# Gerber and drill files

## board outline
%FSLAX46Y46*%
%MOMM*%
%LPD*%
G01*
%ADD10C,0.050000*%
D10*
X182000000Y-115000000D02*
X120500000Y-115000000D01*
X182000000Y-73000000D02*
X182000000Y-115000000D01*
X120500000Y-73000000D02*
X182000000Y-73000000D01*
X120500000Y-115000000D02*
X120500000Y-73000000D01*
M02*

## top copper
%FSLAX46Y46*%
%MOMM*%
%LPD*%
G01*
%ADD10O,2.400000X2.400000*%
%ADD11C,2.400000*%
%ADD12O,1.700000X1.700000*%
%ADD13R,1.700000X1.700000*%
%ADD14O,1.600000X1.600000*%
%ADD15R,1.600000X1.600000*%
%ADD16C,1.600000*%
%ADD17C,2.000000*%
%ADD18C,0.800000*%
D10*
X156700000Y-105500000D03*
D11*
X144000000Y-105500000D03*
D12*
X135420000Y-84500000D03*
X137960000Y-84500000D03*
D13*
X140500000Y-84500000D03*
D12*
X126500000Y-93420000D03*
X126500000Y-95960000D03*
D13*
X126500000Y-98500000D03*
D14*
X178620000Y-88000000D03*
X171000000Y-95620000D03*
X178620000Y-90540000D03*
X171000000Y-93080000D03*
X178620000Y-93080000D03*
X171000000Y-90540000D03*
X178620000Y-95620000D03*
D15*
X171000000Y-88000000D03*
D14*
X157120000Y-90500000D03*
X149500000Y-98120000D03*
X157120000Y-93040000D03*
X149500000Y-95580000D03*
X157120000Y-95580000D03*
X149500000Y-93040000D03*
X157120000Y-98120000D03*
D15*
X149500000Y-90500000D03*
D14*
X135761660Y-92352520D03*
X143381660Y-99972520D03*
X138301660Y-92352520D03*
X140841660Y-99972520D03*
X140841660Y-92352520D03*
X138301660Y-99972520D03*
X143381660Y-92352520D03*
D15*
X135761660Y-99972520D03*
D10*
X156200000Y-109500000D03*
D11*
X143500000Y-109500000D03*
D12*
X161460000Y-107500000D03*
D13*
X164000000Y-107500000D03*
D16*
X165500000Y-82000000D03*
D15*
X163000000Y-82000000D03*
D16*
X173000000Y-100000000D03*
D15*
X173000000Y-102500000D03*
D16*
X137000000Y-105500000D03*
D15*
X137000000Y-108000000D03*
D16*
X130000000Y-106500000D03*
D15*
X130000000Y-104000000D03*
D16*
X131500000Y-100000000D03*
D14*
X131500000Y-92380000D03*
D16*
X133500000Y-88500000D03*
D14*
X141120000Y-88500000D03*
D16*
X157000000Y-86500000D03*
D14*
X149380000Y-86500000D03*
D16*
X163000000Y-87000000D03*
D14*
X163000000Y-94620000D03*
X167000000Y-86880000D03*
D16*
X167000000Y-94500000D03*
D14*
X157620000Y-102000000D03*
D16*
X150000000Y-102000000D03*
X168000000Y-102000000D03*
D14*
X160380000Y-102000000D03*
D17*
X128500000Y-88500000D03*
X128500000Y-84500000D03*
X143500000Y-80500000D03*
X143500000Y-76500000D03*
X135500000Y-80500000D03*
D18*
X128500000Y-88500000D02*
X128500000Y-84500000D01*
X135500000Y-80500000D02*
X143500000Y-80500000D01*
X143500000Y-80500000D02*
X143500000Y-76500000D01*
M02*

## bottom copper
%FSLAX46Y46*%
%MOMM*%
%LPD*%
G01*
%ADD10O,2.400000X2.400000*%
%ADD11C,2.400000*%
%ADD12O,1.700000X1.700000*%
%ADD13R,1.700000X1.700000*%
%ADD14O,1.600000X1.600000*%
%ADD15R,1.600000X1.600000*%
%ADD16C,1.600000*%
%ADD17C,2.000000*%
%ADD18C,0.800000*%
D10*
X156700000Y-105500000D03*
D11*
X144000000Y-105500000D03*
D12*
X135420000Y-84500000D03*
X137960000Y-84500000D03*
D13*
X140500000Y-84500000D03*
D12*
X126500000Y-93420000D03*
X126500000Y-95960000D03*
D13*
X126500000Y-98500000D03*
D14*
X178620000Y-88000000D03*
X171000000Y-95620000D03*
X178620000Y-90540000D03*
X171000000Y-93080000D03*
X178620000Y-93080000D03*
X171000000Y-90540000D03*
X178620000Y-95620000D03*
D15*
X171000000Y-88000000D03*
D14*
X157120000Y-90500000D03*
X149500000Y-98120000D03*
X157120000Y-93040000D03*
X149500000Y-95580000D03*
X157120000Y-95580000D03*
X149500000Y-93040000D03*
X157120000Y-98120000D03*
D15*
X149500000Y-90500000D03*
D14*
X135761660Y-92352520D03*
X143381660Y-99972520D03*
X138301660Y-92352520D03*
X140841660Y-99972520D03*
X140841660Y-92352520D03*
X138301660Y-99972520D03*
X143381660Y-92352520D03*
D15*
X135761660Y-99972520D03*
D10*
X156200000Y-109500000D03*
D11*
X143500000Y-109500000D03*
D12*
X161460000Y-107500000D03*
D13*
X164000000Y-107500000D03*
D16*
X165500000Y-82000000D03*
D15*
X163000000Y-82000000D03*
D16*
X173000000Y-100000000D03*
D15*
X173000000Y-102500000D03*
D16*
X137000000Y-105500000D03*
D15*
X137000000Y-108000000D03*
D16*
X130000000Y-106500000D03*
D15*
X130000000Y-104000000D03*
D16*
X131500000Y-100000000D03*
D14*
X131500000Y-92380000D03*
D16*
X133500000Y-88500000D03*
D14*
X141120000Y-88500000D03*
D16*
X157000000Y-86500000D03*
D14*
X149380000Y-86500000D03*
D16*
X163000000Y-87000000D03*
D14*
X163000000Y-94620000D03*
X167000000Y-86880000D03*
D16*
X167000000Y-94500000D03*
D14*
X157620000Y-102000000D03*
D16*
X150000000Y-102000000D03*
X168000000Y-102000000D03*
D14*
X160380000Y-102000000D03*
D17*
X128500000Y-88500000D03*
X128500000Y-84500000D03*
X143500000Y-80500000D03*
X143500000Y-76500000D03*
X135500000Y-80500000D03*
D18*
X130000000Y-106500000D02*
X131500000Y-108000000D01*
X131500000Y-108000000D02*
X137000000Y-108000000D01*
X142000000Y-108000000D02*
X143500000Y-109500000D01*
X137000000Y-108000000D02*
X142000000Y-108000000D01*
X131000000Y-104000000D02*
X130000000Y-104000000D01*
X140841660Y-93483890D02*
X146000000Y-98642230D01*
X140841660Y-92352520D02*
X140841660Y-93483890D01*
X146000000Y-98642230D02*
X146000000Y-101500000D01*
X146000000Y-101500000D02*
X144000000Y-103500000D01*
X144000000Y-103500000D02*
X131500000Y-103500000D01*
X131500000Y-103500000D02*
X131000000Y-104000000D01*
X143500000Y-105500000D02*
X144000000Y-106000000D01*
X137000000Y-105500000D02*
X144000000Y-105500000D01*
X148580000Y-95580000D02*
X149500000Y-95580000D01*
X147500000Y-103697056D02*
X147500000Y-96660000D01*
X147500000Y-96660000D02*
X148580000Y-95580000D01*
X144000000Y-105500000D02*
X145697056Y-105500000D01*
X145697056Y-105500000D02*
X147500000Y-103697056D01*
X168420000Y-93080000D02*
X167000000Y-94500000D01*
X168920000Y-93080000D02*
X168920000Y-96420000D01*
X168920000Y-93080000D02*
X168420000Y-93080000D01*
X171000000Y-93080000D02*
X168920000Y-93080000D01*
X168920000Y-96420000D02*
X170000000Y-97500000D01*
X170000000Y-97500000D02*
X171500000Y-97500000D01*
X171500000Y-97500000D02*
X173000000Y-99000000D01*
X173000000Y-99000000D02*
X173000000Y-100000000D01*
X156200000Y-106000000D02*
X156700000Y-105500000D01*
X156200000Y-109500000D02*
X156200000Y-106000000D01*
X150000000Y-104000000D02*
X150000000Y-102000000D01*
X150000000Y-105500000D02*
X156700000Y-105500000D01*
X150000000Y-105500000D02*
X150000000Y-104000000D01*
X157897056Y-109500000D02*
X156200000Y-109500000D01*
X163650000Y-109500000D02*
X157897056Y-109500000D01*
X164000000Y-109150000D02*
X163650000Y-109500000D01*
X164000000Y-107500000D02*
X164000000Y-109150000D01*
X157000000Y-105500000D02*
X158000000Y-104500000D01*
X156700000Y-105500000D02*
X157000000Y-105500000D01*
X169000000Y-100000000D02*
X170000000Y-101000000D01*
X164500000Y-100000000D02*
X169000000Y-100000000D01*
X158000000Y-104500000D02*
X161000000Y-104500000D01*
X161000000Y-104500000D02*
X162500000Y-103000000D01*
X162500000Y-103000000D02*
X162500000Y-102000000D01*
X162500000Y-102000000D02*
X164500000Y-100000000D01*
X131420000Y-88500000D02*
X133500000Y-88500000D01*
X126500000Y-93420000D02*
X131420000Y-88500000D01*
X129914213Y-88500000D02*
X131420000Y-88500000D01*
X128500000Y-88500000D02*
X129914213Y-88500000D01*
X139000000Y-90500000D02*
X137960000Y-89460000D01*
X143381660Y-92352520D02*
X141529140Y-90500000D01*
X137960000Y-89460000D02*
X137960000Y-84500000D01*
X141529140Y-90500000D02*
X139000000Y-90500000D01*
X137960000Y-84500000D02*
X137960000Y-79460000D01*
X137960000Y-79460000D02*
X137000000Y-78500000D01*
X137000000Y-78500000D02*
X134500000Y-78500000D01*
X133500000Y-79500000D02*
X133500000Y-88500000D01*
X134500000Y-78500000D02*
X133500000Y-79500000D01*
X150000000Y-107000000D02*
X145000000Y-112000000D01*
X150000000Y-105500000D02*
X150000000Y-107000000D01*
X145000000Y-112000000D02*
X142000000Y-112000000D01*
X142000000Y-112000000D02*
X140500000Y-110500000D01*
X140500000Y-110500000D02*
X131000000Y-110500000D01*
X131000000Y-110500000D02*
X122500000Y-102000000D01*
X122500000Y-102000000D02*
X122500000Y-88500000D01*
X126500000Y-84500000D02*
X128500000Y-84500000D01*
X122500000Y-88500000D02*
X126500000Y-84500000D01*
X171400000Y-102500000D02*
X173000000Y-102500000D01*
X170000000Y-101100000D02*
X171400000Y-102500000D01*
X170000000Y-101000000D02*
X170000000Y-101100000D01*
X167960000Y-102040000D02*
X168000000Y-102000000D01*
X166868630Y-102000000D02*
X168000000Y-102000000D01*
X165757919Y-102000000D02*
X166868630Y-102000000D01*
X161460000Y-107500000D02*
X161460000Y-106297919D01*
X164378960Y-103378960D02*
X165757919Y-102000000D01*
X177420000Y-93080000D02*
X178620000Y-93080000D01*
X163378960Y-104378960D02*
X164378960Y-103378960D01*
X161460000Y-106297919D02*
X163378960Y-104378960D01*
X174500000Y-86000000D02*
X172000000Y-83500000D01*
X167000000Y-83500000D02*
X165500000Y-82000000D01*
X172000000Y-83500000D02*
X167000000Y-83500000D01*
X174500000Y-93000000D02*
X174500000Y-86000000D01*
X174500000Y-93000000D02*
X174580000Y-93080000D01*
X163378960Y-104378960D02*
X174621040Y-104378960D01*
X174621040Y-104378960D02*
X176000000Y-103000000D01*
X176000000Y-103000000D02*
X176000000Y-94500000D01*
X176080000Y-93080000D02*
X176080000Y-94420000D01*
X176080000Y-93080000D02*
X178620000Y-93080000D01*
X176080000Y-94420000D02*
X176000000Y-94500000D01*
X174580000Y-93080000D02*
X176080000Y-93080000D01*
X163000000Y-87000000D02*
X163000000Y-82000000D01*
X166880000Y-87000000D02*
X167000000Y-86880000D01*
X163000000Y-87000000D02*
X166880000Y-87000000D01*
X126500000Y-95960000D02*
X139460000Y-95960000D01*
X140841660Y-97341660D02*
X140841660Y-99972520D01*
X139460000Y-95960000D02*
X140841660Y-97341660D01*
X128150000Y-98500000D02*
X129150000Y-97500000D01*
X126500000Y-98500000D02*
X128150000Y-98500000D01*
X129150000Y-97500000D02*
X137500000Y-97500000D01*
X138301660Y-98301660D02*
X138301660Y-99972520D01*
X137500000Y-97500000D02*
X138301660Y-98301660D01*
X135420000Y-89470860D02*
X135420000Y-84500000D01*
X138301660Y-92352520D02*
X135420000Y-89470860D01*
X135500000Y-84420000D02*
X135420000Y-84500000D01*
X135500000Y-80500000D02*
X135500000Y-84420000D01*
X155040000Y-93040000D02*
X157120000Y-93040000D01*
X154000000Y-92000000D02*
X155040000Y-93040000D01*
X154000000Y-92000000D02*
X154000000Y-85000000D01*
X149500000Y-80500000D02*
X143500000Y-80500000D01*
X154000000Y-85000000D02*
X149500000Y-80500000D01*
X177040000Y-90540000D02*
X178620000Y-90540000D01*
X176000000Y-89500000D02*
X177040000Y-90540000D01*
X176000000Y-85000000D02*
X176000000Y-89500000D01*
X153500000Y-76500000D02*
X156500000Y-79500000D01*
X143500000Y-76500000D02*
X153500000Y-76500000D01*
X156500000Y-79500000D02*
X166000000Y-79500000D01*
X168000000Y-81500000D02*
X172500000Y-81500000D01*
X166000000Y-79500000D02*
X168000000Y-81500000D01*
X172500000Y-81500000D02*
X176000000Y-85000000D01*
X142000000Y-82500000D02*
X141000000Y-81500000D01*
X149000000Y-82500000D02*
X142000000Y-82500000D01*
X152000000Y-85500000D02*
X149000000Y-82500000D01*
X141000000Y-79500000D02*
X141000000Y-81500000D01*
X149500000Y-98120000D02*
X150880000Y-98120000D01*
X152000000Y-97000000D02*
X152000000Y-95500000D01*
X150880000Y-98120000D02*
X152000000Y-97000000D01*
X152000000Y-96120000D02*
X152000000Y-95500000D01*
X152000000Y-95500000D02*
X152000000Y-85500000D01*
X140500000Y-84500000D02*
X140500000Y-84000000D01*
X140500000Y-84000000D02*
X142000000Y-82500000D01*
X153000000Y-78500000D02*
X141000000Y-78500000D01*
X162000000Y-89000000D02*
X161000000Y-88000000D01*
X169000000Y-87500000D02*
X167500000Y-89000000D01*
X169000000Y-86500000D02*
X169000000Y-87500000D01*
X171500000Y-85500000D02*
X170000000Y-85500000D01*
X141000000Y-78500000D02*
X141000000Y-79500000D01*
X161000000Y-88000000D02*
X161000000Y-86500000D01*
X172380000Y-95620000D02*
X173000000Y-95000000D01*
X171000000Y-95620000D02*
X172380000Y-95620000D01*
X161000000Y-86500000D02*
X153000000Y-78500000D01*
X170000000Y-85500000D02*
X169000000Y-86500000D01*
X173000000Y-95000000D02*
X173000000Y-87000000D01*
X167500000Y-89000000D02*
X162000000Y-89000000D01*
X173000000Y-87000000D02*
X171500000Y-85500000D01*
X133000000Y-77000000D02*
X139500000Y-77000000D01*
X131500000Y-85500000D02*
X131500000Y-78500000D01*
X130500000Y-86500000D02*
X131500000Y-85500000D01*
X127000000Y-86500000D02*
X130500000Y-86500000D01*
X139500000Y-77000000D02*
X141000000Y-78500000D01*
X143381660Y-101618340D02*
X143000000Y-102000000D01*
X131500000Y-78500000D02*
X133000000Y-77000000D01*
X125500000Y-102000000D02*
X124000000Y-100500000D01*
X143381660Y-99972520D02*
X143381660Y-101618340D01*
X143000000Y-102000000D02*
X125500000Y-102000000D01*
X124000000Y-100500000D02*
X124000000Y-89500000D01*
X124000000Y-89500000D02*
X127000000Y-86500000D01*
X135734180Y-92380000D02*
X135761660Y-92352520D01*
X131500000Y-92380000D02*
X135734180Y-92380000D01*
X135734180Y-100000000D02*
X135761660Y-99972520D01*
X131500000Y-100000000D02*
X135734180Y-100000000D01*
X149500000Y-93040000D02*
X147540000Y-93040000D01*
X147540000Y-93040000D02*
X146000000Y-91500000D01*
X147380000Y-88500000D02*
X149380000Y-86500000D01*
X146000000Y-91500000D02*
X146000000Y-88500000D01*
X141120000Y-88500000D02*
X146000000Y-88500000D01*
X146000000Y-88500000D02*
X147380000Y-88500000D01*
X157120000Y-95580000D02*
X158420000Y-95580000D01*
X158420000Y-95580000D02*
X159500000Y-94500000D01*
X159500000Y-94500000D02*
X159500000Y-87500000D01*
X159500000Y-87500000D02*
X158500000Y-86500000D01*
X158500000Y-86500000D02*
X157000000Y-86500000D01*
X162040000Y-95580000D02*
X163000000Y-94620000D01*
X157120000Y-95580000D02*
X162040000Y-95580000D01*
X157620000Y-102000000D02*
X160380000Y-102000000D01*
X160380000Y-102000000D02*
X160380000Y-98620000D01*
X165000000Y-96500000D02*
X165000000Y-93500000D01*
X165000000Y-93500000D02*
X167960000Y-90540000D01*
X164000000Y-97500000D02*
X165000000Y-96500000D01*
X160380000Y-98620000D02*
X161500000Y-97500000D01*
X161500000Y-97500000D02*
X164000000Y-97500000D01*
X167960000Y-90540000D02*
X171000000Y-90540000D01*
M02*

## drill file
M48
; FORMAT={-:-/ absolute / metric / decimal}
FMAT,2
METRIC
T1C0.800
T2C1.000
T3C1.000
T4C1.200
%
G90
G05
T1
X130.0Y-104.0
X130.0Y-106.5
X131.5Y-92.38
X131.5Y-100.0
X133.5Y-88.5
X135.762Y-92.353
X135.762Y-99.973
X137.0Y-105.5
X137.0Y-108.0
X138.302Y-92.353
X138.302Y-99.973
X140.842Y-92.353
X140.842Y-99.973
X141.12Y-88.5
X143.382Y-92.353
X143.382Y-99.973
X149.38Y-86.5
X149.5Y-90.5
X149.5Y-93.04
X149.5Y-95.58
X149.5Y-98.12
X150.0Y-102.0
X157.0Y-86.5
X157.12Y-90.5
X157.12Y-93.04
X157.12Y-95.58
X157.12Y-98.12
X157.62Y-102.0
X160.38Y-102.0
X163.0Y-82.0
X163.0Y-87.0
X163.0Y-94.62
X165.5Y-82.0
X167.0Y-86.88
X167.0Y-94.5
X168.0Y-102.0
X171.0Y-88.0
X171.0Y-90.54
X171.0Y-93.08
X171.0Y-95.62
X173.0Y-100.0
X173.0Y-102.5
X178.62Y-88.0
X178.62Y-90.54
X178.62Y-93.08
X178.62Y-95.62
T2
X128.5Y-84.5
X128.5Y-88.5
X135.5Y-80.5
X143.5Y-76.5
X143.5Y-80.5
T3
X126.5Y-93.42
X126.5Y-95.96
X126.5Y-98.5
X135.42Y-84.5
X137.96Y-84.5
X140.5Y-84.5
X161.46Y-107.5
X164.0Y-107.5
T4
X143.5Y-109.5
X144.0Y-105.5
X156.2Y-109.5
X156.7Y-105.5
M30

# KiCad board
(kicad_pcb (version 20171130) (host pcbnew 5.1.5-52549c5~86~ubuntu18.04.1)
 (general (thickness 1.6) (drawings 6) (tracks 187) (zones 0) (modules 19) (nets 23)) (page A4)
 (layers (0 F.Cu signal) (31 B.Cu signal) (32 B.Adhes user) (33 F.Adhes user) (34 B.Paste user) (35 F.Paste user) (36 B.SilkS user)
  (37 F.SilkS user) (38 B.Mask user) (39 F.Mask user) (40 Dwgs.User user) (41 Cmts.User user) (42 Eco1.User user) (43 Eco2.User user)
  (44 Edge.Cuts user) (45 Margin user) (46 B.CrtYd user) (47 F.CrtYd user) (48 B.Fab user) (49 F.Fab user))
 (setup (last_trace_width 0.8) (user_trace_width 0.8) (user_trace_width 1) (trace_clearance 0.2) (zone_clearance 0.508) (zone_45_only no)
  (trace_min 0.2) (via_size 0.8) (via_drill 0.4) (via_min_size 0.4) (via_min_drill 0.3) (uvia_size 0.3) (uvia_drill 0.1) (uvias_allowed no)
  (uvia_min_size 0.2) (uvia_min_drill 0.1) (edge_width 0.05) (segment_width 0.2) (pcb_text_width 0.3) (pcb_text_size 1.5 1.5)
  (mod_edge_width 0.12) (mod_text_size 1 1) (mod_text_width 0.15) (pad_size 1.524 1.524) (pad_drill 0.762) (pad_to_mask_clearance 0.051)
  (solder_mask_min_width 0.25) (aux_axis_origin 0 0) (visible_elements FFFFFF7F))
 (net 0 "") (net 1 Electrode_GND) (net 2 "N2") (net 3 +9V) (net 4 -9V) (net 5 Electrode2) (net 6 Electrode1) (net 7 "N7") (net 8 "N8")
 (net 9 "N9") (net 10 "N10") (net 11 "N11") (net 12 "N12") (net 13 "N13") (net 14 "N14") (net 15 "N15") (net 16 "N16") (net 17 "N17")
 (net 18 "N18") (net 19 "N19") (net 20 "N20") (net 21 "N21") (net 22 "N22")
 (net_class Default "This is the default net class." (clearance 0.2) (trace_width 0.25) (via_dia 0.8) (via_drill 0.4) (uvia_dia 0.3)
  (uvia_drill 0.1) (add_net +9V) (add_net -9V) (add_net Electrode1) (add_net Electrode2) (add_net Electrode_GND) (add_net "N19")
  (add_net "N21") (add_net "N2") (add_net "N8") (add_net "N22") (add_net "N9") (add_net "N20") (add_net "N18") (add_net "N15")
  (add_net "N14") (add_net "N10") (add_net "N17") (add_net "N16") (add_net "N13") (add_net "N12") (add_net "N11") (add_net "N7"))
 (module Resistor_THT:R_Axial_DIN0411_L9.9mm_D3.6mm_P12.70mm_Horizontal (layer F.Cu) (at 144 105.5)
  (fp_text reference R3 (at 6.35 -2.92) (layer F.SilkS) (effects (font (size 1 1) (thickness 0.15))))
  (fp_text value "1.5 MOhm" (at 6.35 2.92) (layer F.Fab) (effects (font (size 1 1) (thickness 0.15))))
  (pad 2 thru_hole oval (at 12.7 0) (size 2.4 2.4) (drill 1.2) (layers *.Cu *.Mask) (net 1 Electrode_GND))
  (pad 1 thru_hole circle (at 0 0) (size 2.4 2.4) (drill 1.2) (layers *.Cu *.Mask) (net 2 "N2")))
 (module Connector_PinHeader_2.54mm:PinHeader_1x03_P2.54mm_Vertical (layer F.Cu) (at 140.5 84.5 270)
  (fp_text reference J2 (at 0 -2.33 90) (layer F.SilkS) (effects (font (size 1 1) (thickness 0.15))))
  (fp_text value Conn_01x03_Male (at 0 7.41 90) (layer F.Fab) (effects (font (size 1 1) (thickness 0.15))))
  (pad 3 thru_hole oval (at 0 5.08 270) (size 1.7 1.7) (drill 1) (layers *.Cu *.Mask) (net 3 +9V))
  (pad 2 thru_hole oval (at 0 2.54 270) (size 1.7 1.7) (drill 1) (layers *.Cu *.Mask) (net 1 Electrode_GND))
  (pad 1 thru_hole rect (at 0 0 270) (size 1.7 1.7) (drill 1) (layers *.Cu *.Mask) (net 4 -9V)))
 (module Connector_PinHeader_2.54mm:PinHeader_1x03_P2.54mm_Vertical (layer F.Cu) (at 126.5 98.5 180)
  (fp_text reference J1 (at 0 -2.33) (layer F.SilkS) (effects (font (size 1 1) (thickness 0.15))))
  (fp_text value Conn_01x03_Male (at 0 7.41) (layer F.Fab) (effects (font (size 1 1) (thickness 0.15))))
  (pad 3 thru_hole oval (at 0 5.08 180) (size 1.7 1.7) (drill 1) (layers *.Cu *.Mask) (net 1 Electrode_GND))
  (pad 2 thru_hole oval (at 0 2.54 180) (size 1.7 1.7) (drill 1) (layers *.Cu *.Mask) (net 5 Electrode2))
  (pad 1 thru_hole rect (at 0 0 180) (size 1.7 1.7) (drill 1) (layers *.Cu *.Mask) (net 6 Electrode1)))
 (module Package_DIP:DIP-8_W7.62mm (layer F.Cu) (at 171 88)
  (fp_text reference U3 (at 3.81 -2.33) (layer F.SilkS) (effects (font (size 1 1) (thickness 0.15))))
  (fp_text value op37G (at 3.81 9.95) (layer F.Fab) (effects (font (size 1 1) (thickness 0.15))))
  (pad 8 thru_hole oval (at 7.62 0) (size 1.6 1.6) (drill 0.8) (layers *.Cu *.Mask) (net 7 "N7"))
  (pad 4 thru_hole oval (at 0 7.62) (size 1.6 1.6) (drill 0.8) (layers *.Cu *.Mask) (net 4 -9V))
  (pad 7 thru_hole oval (at 7.62 2.54) (size 1.6 1.6) (drill 0.8) (layers *.Cu *.Mask) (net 3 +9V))
  (pad 3 thru_hole oval (at 0 5.08) (size 1.6 1.6) (drill 0.8) (layers *.Cu *.Mask) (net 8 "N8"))
  (pad 6 thru_hole oval (at 7.62 5.08) (size 1.6 1.6) (drill 0.8) (layers *.Cu *.Mask) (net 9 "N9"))
  (pad 2 thru_hole oval (at 0 2.54) (size 1.6 1.6) (drill 0.8) (layers *.Cu *.Mask) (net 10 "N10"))
  (pad 5 thru_hole oval (at 7.62 7.62) (size 1.6 1.6) (drill 0.8) (layers *.Cu *.Mask) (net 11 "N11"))
  (pad 1 thru_hole rect (at 0 0) (size 1.6 1.6) (drill 0.8) (layers *.Cu *.Mask) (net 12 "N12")))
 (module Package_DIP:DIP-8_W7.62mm (layer F.Cu) (at 149.5 90.5)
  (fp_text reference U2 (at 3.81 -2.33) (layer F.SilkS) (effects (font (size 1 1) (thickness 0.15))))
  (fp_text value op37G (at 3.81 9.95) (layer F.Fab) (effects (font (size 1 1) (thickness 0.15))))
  (pad 8 thru_hole oval (at 7.62 0) (size 1.6 1.6) (drill 0.8) (layers *.Cu *.Mask) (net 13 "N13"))
  (pad 4 thru_hole oval (at 0 7.62) (size 1.6 1.6) (drill 0.8) (layers *.Cu *.Mask) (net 4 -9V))
  (pad 7 thru_hole oval (at 7.62 2.54) (size 1.6 1.6) (drill 0.8) (layers *.Cu *.Mask) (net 3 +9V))
  (pad 3 thru_hole oval (at 0 5.08) (size 1.6 1.6) (drill 0.8) (layers *.Cu *.Mask) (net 2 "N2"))
  (pad 6 thru_hole oval (at 7.62 5.08) (size 1.6 1.6) (drill 0.8) (layers *.Cu *.Mask) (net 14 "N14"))
  (pad 2 thru_hole oval (at 0 2.54) (size 1.6 1.6) (drill 0.8) (layers *.Cu *.Mask) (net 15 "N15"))
  (pad 5 thru_hole oval (at 7.62 7.62) (size 1.6 1.6) (drill 0.8) (layers *.Cu *.Mask) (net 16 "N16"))
  (pad 1 thru_hole rect (at 0 0) (size 1.6 1.6) (drill 0.8) (layers *.Cu *.Mask) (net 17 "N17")))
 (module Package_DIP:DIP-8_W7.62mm (layer F.Cu) (at 135.76166 99.97252 90)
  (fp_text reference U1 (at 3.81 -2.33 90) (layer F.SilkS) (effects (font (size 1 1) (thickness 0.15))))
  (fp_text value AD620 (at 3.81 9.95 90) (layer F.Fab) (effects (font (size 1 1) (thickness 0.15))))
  (pad 8 thru_hole oval (at 7.62 0 90) (size 1.6 1.6) (drill 0.8) (layers *.Cu *.Mask) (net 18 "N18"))
  (pad 4 thru_hole oval (at 0 7.62 90) (size 1.6 1.6) (drill 0.8) (layers *.Cu *.Mask) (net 4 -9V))
  (pad 7 thru_hole oval (at 7.62 2.54 90) (size 1.6 1.6) (drill 0.8) (layers *.Cu *.Mask) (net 3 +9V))
  (pad 3 thru_hole oval (at 0 5.08 90) (size 1.6 1.6) (drill 0.8) (layers *.Cu *.Mask) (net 5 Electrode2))
  (pad 6 thru_hole oval (at 7.62 5.08 90) (size 1.6 1.6) (drill 0.8) (layers *.Cu *.Mask) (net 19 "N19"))
  (pad 2 thru_hole oval (at 0 2.54 90) (size 1.6 1.6) (drill 0.8) (layers *.Cu *.Mask) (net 6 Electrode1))
  (pad 5 thru_hole oval (at 7.62 7.62 90) (size 1.6 1.6) (drill 0.8) (layers *.Cu *.Mask) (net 1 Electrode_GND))
  (pad 1 thru_hole rect (at 0 0 90) (size 1.6 1.6) (drill 0.8) (layers *.Cu *.Mask) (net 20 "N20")))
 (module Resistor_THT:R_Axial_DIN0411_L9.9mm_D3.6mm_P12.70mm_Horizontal (layer F.Cu) (at 143.5 109.5)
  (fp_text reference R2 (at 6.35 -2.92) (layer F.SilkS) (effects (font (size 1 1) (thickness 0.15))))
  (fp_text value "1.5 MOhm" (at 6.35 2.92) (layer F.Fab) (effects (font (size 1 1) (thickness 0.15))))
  (pad 2 thru_hole oval (at 12.7 0) (size 2.4 2.4) (drill 1.2) (layers *.Cu *.Mask) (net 1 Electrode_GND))
  (pad 1 thru_hole circle (at 0 0) (size 2.4 2.4) (drill 1.2) (layers *.Cu *.Mask) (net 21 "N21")))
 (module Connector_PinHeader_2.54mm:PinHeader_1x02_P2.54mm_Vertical (layer F.Cu) (at 164 107.5 270)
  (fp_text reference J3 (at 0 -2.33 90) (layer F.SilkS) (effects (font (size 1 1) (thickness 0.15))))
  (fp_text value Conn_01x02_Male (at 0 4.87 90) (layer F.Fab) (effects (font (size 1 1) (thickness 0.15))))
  (pad 2 thru_hole oval (at 0 2.54 270) (size 1.7 1.7) (drill 1) (layers *.Cu *.Mask) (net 9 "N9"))
  (pad 1 thru_hole rect (at 0 0 270) (size 1.7 1.7) (drill 1) (layers *.Cu *.Mask) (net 1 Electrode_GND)))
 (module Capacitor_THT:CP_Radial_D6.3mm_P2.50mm (layer F.Cu) (at 163 82)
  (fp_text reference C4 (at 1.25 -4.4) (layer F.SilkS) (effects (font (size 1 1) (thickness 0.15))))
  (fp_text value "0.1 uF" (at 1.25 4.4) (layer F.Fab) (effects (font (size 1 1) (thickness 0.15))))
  (pad 2 thru_hole circle (at 2.5 0) (size 1.6 1.6) (drill 0.8) (layers *.Cu *.Mask) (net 9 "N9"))
  (pad 1 thru_hole rect (at 0 0) (size 1.6 1.6) (drill 0.8) (layers *.Cu *.Mask) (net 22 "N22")))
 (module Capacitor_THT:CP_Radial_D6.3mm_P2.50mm (layer F.Cu) (at 173 102.5 90)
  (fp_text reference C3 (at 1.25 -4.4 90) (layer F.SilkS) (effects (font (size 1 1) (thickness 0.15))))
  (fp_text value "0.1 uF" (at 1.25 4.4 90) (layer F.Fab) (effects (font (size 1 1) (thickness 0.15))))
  (pad 2 thru_hole circle (at 2.5 0 90) (size 1.6 1.6) (drill 0.8) (layers *.Cu *.Mask) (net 8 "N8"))
  (pad 1 thru_hole rect (at 0 0 90) (size 1.6 1.6) (drill 0.8) (layers *.Cu *.Mask) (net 1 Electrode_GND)))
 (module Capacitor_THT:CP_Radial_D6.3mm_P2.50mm (layer F.Cu) (at 137 108 90)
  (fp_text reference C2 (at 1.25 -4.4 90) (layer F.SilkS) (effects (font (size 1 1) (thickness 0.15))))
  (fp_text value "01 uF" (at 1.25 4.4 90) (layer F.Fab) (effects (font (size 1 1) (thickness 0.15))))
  (pad 2 thru_hole circle (at 2.5 0 90) (size 1.6 1.6) (drill 0.8) (layers *.Cu *.Mask) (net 2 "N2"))
  (pad 1 thru_hole rect (at 0 0 90) (size 1.6 1.6) (drill 0.8) (layers *.Cu *.Mask) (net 21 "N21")))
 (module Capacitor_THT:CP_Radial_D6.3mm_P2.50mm (layer F.Cu) (at 130 104 270)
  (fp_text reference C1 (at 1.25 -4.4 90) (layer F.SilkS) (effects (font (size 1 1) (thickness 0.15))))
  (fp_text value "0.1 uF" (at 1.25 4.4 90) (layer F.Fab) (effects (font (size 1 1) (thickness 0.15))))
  (pad 2 thru_hole circle (at 2.5 0 270) (size 1.6 1.6) (drill 0.8) (layers *.Cu *.Mask) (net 21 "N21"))
  (pad 1 thru_hole rect (at 0 0 270) (size 1.6 1.6) (drill 0.8) (layers *.Cu *.Mask) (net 19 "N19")))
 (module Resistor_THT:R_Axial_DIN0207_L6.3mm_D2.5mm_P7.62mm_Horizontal (layer F.Cu) (at 131.5 100 90)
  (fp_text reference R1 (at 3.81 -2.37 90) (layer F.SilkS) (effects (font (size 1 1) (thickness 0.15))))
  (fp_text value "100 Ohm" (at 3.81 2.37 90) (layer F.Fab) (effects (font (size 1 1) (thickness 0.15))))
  (pad 1 thru_hole circle (at 0 0 90) (size 1.6 1.6) (drill 0.8) (layers *.Cu *.Mask) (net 20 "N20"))
  (pad 2 thru_hole oval (at 7.62 0 90) (size 1.6 1.6) (drill 0.8) (layers *.Cu *.Mask) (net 18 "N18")))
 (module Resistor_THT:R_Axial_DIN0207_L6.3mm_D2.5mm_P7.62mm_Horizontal (layer F.Cu) (at 133.5 88.5)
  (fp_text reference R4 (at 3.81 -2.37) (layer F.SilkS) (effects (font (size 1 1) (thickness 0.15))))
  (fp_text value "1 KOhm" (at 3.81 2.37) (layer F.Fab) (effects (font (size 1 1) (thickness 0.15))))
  (pad 1 thru_hole circle (at 0 0) (size 1.6 1.6) (drill 0.8) (layers *.Cu *.Mask) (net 1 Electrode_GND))
  (pad 2 thru_hole oval (at 7.62 0) (size 1.6 1.6) (drill 0.8) (layers *.Cu *.Mask) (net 15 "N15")))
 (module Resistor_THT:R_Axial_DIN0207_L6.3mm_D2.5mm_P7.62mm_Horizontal (layer F.Cu) (at 157 86.5 180)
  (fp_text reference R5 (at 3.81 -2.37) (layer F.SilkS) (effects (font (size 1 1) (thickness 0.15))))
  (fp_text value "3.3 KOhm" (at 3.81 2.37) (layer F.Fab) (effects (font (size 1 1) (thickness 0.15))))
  (pad 1 thru_hole circle (at 0 0 180) (size 1.6 1.6) (drill 0.8) (layers *.Cu *.Mask) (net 14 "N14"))
  (pad 2 thru_hole oval (at 7.62 0 180) (size 1.6 1.6) (drill 0.8) (layers *.Cu *.Mask) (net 15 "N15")))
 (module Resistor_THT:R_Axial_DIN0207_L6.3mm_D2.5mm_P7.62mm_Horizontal (layer F.Cu) (at 163 87 270)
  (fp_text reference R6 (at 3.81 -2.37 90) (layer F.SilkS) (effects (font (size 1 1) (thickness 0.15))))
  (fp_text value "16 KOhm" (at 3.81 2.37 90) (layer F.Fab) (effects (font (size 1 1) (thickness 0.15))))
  (pad 1 thru_hole circle (at 0 0 270) (size 1.6 1.6) (drill 0.8) (layers *.Cu *.Mask) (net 22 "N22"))
  (pad 2 thru_hole oval (at 7.62 0 270) (size 1.6 1.6) (drill 0.8) (layers *.Cu *.Mask) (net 14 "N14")))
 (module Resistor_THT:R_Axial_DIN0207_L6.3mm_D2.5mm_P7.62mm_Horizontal (layer F.Cu) (at 167 94.5 90)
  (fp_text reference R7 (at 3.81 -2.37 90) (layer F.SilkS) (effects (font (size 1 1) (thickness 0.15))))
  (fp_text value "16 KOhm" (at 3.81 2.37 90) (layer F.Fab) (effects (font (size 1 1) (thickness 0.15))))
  (pad 2 thru_hole oval (at 7.62 0 90) (size 1.6 1.6) (drill 0.8) (layers *.Cu *.Mask) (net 22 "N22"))
  (pad 1 thru_hole circle (at 0 0 90) (size 1.6 1.6) (drill 0.8) (layers *.Cu *.Mask) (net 8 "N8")))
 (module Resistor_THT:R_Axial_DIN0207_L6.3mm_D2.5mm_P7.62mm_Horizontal (layer F.Cu) (at 150 102)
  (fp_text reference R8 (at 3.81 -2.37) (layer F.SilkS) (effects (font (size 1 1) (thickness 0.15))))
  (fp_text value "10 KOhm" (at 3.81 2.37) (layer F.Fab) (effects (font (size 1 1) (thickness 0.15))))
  (pad 2 thru_hole oval (at 7.62 0) (size 1.6 1.6) (drill 0.8) (layers *.Cu *.Mask) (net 10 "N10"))
  (pad 1 thru_hole circle (at 0 0) (size 1.6 1.6) (drill 0.8) (layers *.Cu *.Mask) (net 1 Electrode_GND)))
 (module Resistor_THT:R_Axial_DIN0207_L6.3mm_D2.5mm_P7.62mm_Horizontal (layer F.Cu) (at 168 102 180)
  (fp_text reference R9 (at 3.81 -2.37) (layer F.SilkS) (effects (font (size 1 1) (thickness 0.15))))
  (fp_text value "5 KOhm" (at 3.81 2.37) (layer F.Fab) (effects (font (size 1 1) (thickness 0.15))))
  (pad 1 thru_hole circle (at 0 0 180) (size 1.6 1.6) (drill 0.8) (layers *.Cu *.Mask) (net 9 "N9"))
  (pad 2 thru_hole oval (at 7.62 0 180) (size 1.6 1.6) (drill 0.8) (layers *.Cu *.Mask) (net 10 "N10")))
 (gr_line (start 182 115) (end 120.5 115) (layer Edge.Cuts) (width 0.05))
 (gr_line (start 182 73) (end 182 115) (layer Edge.Cuts) (width 0.05))
 (gr_line (start 120.5 73) (end 182 73) (layer Edge.Cuts) (width 0.05))
 (gr_line (start 120.5 115) (end 120.5 73) (layer Edge.Cuts) (width 0.05))
 (segment (start 130 106.5) (end 131.5 108) (width 0.8) (layer B.Cu) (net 21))
 (segment (start 131.5 108) (end 137 108) (width 0.8) (layer B.Cu) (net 21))
 (segment (start 142 108) (end 143.5 109.5) (width 0.8) (layer B.Cu) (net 21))
 (segment (start 137 108) (end 142 108) (width 0.8) (layer B.Cu) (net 21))
 (segment (start 131 104) (end 130 104) (width 0.8) (layer B.Cu) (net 19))
 (segment (start 140.84166 93.48389) (end 146 98.64223) (width 0.8) (layer B.Cu) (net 19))
 (segment (start 140.84166 92.35252) (end 140.84166 93.48389) (width 0.8) (layer B.Cu) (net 19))
 (segment (start 146 98.64223) (end 146 101.5) (width 0.8) (layer B.Cu) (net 19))
 (segment (start 146 101.5) (end 144 103.5) (width 0.8) (layer B.Cu) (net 19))
 (segment (start 144 103.5) (end 131.5 103.5) (width 0.8) (layer B.Cu) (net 19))
 (segment (start 131.5 103.5) (end 131 104) (width 0.8) (layer B.Cu) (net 19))
 (segment (start 143.5 105.5) (end 144 106) (width 0.8) (layer B.Cu) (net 2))
 (segment (start 137 105.5) (end 144 105.5) (width 0.8) (layer B.Cu) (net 2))
 (segment (start 148.58 95.58) (end 149.5 95.58) (width 0.8) (layer B.Cu) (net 2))
 (segment (start 147.5 103.697056) (end 147.5 96.66) (width 0.8) (layer B.Cu) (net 2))
 (segment (start 147.5 96.66) (end 148.58 95.58) (width 0.8) (layer B.Cu) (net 2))
 (segment (start 144 105.5) (end 145.697056 105.5) (width 0.8) (layer B.Cu) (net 2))
 (segment (start 145.697056 105.5) (end 147.5 103.697056) (width 0.8) (layer B.Cu) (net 2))
 (segment (start 168.42 93.08) (end 167 94.5) (width 0.8) (layer B.Cu) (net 8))
 (segment (start 168.92 93.08) (end 168.92 96.42) (width 0.8) (layer B.Cu) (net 8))
 (segment (start 168.92 93.08) (end 168.42 93.08) (width 0.8) (layer B.Cu) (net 8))
 (segment (start 171 93.08) (end 168.92 93.08) (width 0.8) (layer B.Cu) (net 8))
 (segment (start 168.92 96.42) (end 170 97.5) (width 0.8) (layer B.Cu) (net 8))
 (segment (start 170 97.5) (end 171.5 97.5) (width 0.8) (layer B.Cu) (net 8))
 (segment (start 171.5 97.5) (end 173 99) (width 0.8) (layer B.Cu) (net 8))
 (segment (start 173 99) (end 173 100) (width 0.8) (layer B.Cu) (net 8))
 (segment (start 156.2 106) (end 156.7 105.5) (width 0.8) (layer B.Cu) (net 1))
 (segment (start 156.2 109.5) (end 156.2 106) (width 0.8) (layer B.Cu) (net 1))
 (segment (start 150 104) (end 150 102) (width 0.8) (layer B.Cu) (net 1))
 (segment (start 150 105.5) (end 156.7 105.5) (width 0.8) (layer B.Cu) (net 1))
 (segment (start 150 105.5) (end 150 104) (width 0.8) (layer B.Cu) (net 1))
 (segment (start 157.897056 109.5) (end 156.2 109.5) (width 0.8) (layer B.Cu) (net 1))
 (segment (start 163.65 109.5) (end 157.897056 109.5) (width 0.8) (layer B.Cu) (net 1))
 (segment (start 164 109.15) (end 163.65 109.5) (width 0.8) (layer B.Cu) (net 1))
 (segment (start 164 107.5) (end 164 109.15) (width 0.8) (layer B.Cu) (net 1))
 (segment (start 157 105.5) (end 158 104.5) (width 0.8) (layer B.Cu) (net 1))
 (segment (start 156.7 105.5) (end 157 105.5) (width 0.8) (layer B.Cu) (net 1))
 (segment (start 169 100) (end 170 101) (width 0.8) (layer B.Cu) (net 1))
 (segment (start 164.5 100) (end 169 100) (width 0.8) (layer B.Cu) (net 1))
 (segment (start 158 104.5) (end 161 104.5) (width 0.8) (layer B.Cu) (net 1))
 (segment (start 161 104.5) (end 162.5 103) (width 0.8) (layer B.Cu) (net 1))
 (segment (start 162.5 103) (end 162.5 102) (width 0.8) (layer B.Cu) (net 1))
 (segment (start 162.5 102) (end 164.5 100) (width 0.8) (layer B.Cu) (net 1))
 (via (at 128.5 88.5) (size 2) (drill 1) (layers F.Cu B.Cu) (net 1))
 (segment (start 131.42 88.5) (end 133.5 88.5) (width 0.8) (layer B.Cu) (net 1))
 (segment (start 126.5 93.42) (end 131.42 88.5) (width 0.8) (layer B.Cu) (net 1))
 (segment (start 129.914213 88.5) (end 131.42 88.5) (width 0.8) (layer B.Cu) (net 1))
 (segment (start 128.5 88.5) (end 129.914213 88.5) (width 0.8) (layer B.Cu) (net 1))
 (segment (start 139 90.5) (end 137.96 89.46) (width 0.8) (layer B.Cu) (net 1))
 (segment (start 143.38166 92.35252) (end 141.52914 90.5) (width 0.8) (layer B.Cu) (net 1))
 (segment (start 137.96 89.46) (end 137.96 84.5) (width 0.8) (layer B.Cu) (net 1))
 (segment (start 141.52914 90.5) (end 139 90.5) (width 0.8) (layer B.Cu) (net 1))
 (segment (start 137.96 84.5) (end 137.96 79.46) (width 0.8) (layer B.Cu) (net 1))
 (segment (start 137.96 79.46) (end 137 78.5) (width 0.8) (layer B.Cu) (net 1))
 (segment (start 137 78.5) (end 134.5 78.5) (width 0.8) (layer B.Cu) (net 1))
 (segment (start 133.5 79.5) (end 133.5 88.5) (width 0.8) (layer B.Cu) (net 1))
 (segment (start 134.5 78.5) (end 133.5 79.5) (width 0.8) (layer B.Cu) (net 1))
 (segment (start 150 107) (end 145 112) (width 0.8) (layer B.Cu) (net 1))
 (segment (start 150 105.5) (end 150 107) (width 0.8) (layer B.Cu) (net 1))
 (segment (start 145 112) (end 142 112) (width 0.8) (layer B.Cu) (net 1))
 (segment (start 142 112) (end 140.5 110.5) (width 0.8) (layer B.Cu) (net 1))
 (segment (start 140.5 110.5) (end 131 110.5) (width 0.8) (layer B.Cu) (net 1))
 (segment (start 131 110.5) (end 122.5 102) (width 0.8) (layer B.Cu) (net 1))
 (via (at 128.5 84.5) (size 2) (drill 1) (layers F.Cu B.Cu) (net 1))
 (segment (start 122.5 102) (end 122.5 88.5) (width 0.8) (layer B.Cu) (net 1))
 (segment (start 126.5 84.5) (end 128.5 84.5) (width 0.8) (layer B.Cu) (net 1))
 (segment (start 122.5 88.5) (end 126.5 84.5) (width 0.8) (layer B.Cu) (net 1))
 (segment (start 128.5 88.5) (end 128.5 84.5) (width 0.8) (layer F.Cu) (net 1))
 (segment (start 171.4 102.5) (end 173 102.5) (width 0.8) (layer B.Cu) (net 1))
 (segment (start 170 101.1) (end 171.4 102.5) (width 0.8) (layer B.Cu) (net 1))
 (segment (start 170 101) (end 170 101.1) (width 0.8) (layer B.Cu) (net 1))
 (segment (start 167.96 102.04) (end 168 102) (width 0.8) (layer B.Cu) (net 9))
 (segment (start 166.86863 102) (end 168 102) (width 0.8) (layer B.Cu) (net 9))
 (segment (start 165.757919 102) (end 166.86863 102) (width 0.8) (layer B.Cu) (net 9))
 (segment (start 161.46 107.5) (end 161.46 106.297919) (width 0.8) (layer B.Cu) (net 9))
 (segment (start 164.37896 103.37896) (end 165.757919 102) (width 0.8) (layer B.Cu) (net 9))
 (segment (start 177.42 93.08) (end 178.62 93.08) (width 0.8) (layer B.Cu) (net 9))
 (segment (start 163.37896 104.37896) (end 164.37896 103.37896) (width 0.8) (layer B.Cu) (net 9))
 (segment (start 161.46 106.297919) (end 163.37896 104.37896) (width 0.8) (layer B.Cu) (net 9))
 (segment (start 174.5 86) (end 172 83.5) (width 0.8) (layer B.Cu) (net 9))
 (segment (start 167 83.5) (end 165.5 82) (width 0.8) (layer B.Cu) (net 9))
 (segment (start 172 83.5) (end 167 83.5) (width 0.8) (layer B.Cu) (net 9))
 (segment (start 174.5 93) (end 174.5 86) (width 0.8) (layer B.Cu) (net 9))
 (segment (start 174.5 93) (end 174.58 93.08) (width 0.8) (layer B.Cu) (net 9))
 (segment (start 163.37896 104.37896) (end 174.62104 104.37896) (width 0.8) (layer B.Cu) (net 9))
 (segment (start 174.62104 104.37896) (end 176 103) (width 0.8) (layer B.Cu) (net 9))
 (segment (start 176 103) (end 176 94.5) (width 0.8) (layer B.Cu) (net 9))
 (segment (start 176.08 93.08) (end 176.08 94.42) (width 0.8) (layer B.Cu) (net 9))
 (segment (start 176.08 93.08) (end 178.62 93.08) (width 0.8) (layer B.Cu) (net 9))
 (segment (start 176.08 94.42) (end 176 94.5) (width 0.8) (layer B.Cu) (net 9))
 (segment (start 174.58 93.08) (end 176.08 93.08) (width 0.8) (layer B.Cu) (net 9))
 (segment (start 163 87) (end 163 82) (width 0.8) (layer B.Cu) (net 22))
 (segment (start 166.88 87) (end 167 86.88) (width 0.8) (layer B.Cu) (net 22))
 (segment (start 163 87) (end 166.88 87) (width 0.8) (layer B.Cu) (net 22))
 (segment (start 126.5 95.96) (end 139.46 95.96) (width 0.8) (layer B.Cu) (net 5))
 (segment (start 140.84166 97.34166) (end 140.84166 99.97252) (width 0.8) (layer B.Cu) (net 5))
 (segment (start 139.46 95.96) (end 140.84166 97.34166) (width 0.8) (layer B.Cu) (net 5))
 (segment (start 128.15 98.5) (end 129.15 97.5) (width 0.8) (layer B.Cu) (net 6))
 (segment (start 126.5 98.5) (end 128.15 98.5) (width 0.8) (layer B.Cu) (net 6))
 (segment (start 129.15 97.5) (end 137.5 97.5) (width 0.8) (layer B.Cu) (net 6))
 (segment (start 138.30166 98.30166) (end 138.30166 99.97252) (width 0.8) (layer B.Cu) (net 6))
 (segment (start 137.5 97.5) (end 138.30166 98.30166) (width 0.8) (layer B.Cu) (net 6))
 (via (at 143.5 80.5) (size 2) (drill 1) (layers F.Cu B.Cu) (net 3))
 (via (at 143.5 76.5) (size 2) (drill 1) (layers F.Cu B.Cu) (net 3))
 (via (at 135.5 80.5) (size 2) (drill 1) (layers F.Cu B.Cu) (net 3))
 (segment (start 135.42 89.47086) (end 135.42 84.5) (width 0.8) (layer B.Cu) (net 3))
 (segment (start 138.30166 92.35252) (end 135.42 89.47086) (width 0.8) (layer B.Cu) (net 3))
 (segment (start 135.5 84.42) (end 135.42 84.5) (width 0.8) (layer B.Cu) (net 3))
 (segment (start 135.5 80.5) (end 135.5 84.42) (width 0.8) (layer B.Cu) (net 3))
 (segment (start 155.04 93.04) (end 157.12 93.04) (width 0.8) (layer B.Cu) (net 3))
 (segment (start 154 92) (end 155.04 93.04) (width 0.8) (layer B.Cu) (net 3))
 (segment (start 154 92) (end 154 85) (width 0.8) (layer B.Cu) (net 3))
 (segment (start 149.5 80.5) (end 143.5 80.5) (width 0.8) (layer B.Cu) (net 3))
 (segment (start 154 85) (end 149.5 80.5) (width 0.8) (layer B.Cu) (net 3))
 (segment (start 177.04 90.54) (end 178.62 90.54) (width 0.8) (layer B.Cu) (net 3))
 (segment (start 176 89.5) (end 177.04 90.54) (width 0.8) (layer B.Cu) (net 3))
 (segment (start 176 85) (end 176 89.5) (width 0.8) (layer B.Cu) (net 3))
 (segment (start 153.5 76.5) (end 156.5 79.5) (width 0.8) (layer B.Cu) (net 3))
 (segment (start 143.5 76.5) (end 153.5 76.5) (width 0.8) (layer B.Cu) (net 3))
 (segment (start 156.5 79.5) (end 166 79.5) (width 0.8) (layer B.Cu) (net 3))
 (segment (start 168 81.5) (end 172.5 81.5) (width 0.8) (layer B.Cu) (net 3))
 (segment (start 166 79.5) (end 168 81.5) (width 0.8) (layer B.Cu) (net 3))
 (segment (start 172.5 81.5) (end 176 85) (width 0.8) (layer B.Cu) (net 3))
 (segment (start 135.5 80.5) (end 143.5 80.5) (width 0.8) (layer F.Cu) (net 3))
 (segment (start 143.5 80.5) (end 143.5 76.5) (width 0.8) (layer F.Cu) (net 3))
 (segment (start 142 82.5) (end 141 81.5) (width 0.8) (layer B.Cu) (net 4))
 (segment (start 149 82.5) (end 142 82.5) (width 0.8) (layer B.Cu) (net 4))
 (segment (start 152 85.5) (end 149 82.5) (width 0.8) (layer B.Cu) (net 4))
 (segment (start 141 79.5) (end 141 81.5) (width 0.8) (layer B.Cu) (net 4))
 (segment (start 149.5 98.12) (end 150.88 98.12) (width 0.8) (layer B.Cu) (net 4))
 (segment (start 152 97) (end 152 95.5) (width 0.8) (layer B.Cu) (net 4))
 (segment (start 150.88 98.12) (end 152 97) (width 0.8) (layer B.Cu) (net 4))
 (segment (start 152 96.12) (end 152 95.5) (width 0.8) (layer B.Cu) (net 4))
 (segment (start 152 95.5) (end 152 85.5) (width 0.8) (layer B.Cu) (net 4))
 (segment (start 140.5 84.5) (end 140.5 84) (width 0.8) (layer B.Cu) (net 4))
 (segment (start 140.5 84) (end 142 82.5) (width 0.8) (layer B.Cu) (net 4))
 (segment (start 153 78.5) (end 141 78.5) (width 0.8) (layer B.Cu) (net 4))
 (segment (start 162 89) (end 161 88) (width 0.8) (layer B.Cu) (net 4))
 (segment (start 169 87.5) (end 167.5 89) (width 0.8) (layer B.Cu) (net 4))
 (segment (start 169 86.5) (end 169 87.5) (width 0.8) (layer B.Cu) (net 4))
 (segment (start 171.5 85.5) (end 170 85.5) (width 0.8) (layer B.Cu) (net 4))
 (segment (start 141 78.5) (end 141 79.5) (width 0.8) (layer B.Cu) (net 4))
 (segment (start 161 88) (end 161 86.5) (width 0.8) (layer B.Cu) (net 4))
 (segment (start 172.38 95.62) (end 173 95) (width 0.8) (layer B.Cu) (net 4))
 (segment (start 171 95.62) (end 172.38 95.62) (width 0.8) (layer B.Cu) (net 4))
 (segment (start 161 86.5) (end 153 78.5) (width 0.8) (layer B.Cu) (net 4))
 (segment (start 170 85.5) (end 169 86.5) (width 0.8) (layer B.Cu) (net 4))
 (segment (start 173 95) (end 173 87) (width 0.8) (layer B.Cu) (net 4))
 (segment (start 167.5 89) (end 162 89) (width 0.8) (layer B.Cu) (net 4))
 (segment (start 173 87) (end 171.5 85.5) (width 0.8) (layer B.Cu) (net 4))
 (segment (start 133 77) (end 139.5 77) (width 0.8) (layer B.Cu) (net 4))
 (segment (start 131.5 85.5) (end 131.5 78.5) (width 0.8) (layer B.Cu) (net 4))
 (segment (start 130.5 86.5) (end 131.5 85.5) (width 0.8) (layer B.Cu) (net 4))
 (segment (start 127 86.5) (end 130.5 86.5) (width 0.8) (layer B.Cu) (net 4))
 (segment (start 139.5 77) (end 141 78.5) (width 0.8) (layer B.Cu) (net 4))
 (segment (start 143.38166 101.61834) (end 143 102) (width 0.8) (layer B.Cu) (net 4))
 (segment (start 131.5 78.5) (end 133 77) (width 0.8) (layer B.Cu) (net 4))
 (segment (start 125.5 102) (end 124 100.5) (width 0.8) (layer B.Cu) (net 4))
 (segment (start 143.38166 99.97252) (end 143.38166 101.61834) (width 0.8) (layer B.Cu) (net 4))
 (segment (start 143 102) (end 125.5 102) (width 0.8) (layer B.Cu) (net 4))
 (segment (start 124 100.5) (end 124 89.5) (width 0.8) (layer B.Cu) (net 4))
 (segment (start 124 89.5) (end 127 86.5) (width 0.8) (layer B.Cu) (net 4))
 (segment (start 135.73418 92.38) (end 135.76166 92.35252) (width 0.8) (layer B.Cu) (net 18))
 (segment (start 131.5 92.38) (end 135.73418 92.38) (width 0.8) (layer B.Cu) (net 18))
 (segment (start 135.73418 100) (end 135.76166 99.97252) (width 0.8) (layer B.Cu) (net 20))
 (segment (start 131.5 100) (end 135.73418 100) (width 0.8) (layer B.Cu) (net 20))
 (segment (start 149.5 93.04) (end 147.54 93.04) (width 0.8) (layer B.Cu) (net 15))
 (segment (start 147.54 93.04) (end 146 91.5) (width 0.8) (layer B.Cu) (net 15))
 (segment (start 147.38 88.5) (end 149.38 86.5) (width 0.8) (layer B.Cu) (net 15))
 (segment (start 146 91.5) (end 146 88.5) (width 0.8) (layer B.Cu) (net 15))
 (segment (start 141.12 88.5) (end 146 88.5) (width 0.8) (layer B.Cu) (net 15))
 (segment (start 146 88.5) (end 147.38 88.5) (width 0.8) (layer B.Cu) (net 15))
 (segment (start 157.12 95.58) (end 158.42 95.58) (width 0.8) (layer B.Cu) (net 14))
 (segment (start 158.42 95.58) (end 159.5 94.5) (width 0.8) (layer B.Cu) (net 14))
 (segment (start 159.5 94.5) (end 159.5 87.5) (width 0.8) (layer B.Cu) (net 14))
 (segment (start 159.5 87.5) (end 158.5 86.5) (width 0.8) (layer B.Cu) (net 14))
 (segment (start 158.5 86.5) (end 157 86.5) (width 0.8) (layer B.Cu) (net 14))
 (segment (start 162.04 95.58) (end 163 94.62) (width 0.8) (layer B.Cu) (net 14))
 (segment (start 157.12 95.58) (end 162.04 95.58) (width 0.8) (layer B.Cu) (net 14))
 (segment (start 157.62 102) (end 160.38 102) (width 0.8) (layer B.Cu) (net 10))
 (segment (start 160.38 102) (end 160.38 98.62) (width 0.8) (layer B.Cu) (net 10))
 (segment (start 165 96.5) (end 165 93.5) (width 0.8) (layer B.Cu) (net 10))
 (segment (start 165 93.5) (end 167.96 90.54) (width 0.8) (layer B.Cu) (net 10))
 (segment (start 164 97.5) (end 165 96.5) (width 0.8) (layer B.Cu) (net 10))
 (segment (start 160.38 98.62) (end 161.5 97.5) (width 0.8) (layer B.Cu) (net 10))
 (segment (start 161.5 97.5) (end 164 97.5) (width 0.8) (layer B.Cu) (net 10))
 (segment (start 167.96 90.54) (end 171 90.54) (width 0.8) (layer B.Cu) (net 10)))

